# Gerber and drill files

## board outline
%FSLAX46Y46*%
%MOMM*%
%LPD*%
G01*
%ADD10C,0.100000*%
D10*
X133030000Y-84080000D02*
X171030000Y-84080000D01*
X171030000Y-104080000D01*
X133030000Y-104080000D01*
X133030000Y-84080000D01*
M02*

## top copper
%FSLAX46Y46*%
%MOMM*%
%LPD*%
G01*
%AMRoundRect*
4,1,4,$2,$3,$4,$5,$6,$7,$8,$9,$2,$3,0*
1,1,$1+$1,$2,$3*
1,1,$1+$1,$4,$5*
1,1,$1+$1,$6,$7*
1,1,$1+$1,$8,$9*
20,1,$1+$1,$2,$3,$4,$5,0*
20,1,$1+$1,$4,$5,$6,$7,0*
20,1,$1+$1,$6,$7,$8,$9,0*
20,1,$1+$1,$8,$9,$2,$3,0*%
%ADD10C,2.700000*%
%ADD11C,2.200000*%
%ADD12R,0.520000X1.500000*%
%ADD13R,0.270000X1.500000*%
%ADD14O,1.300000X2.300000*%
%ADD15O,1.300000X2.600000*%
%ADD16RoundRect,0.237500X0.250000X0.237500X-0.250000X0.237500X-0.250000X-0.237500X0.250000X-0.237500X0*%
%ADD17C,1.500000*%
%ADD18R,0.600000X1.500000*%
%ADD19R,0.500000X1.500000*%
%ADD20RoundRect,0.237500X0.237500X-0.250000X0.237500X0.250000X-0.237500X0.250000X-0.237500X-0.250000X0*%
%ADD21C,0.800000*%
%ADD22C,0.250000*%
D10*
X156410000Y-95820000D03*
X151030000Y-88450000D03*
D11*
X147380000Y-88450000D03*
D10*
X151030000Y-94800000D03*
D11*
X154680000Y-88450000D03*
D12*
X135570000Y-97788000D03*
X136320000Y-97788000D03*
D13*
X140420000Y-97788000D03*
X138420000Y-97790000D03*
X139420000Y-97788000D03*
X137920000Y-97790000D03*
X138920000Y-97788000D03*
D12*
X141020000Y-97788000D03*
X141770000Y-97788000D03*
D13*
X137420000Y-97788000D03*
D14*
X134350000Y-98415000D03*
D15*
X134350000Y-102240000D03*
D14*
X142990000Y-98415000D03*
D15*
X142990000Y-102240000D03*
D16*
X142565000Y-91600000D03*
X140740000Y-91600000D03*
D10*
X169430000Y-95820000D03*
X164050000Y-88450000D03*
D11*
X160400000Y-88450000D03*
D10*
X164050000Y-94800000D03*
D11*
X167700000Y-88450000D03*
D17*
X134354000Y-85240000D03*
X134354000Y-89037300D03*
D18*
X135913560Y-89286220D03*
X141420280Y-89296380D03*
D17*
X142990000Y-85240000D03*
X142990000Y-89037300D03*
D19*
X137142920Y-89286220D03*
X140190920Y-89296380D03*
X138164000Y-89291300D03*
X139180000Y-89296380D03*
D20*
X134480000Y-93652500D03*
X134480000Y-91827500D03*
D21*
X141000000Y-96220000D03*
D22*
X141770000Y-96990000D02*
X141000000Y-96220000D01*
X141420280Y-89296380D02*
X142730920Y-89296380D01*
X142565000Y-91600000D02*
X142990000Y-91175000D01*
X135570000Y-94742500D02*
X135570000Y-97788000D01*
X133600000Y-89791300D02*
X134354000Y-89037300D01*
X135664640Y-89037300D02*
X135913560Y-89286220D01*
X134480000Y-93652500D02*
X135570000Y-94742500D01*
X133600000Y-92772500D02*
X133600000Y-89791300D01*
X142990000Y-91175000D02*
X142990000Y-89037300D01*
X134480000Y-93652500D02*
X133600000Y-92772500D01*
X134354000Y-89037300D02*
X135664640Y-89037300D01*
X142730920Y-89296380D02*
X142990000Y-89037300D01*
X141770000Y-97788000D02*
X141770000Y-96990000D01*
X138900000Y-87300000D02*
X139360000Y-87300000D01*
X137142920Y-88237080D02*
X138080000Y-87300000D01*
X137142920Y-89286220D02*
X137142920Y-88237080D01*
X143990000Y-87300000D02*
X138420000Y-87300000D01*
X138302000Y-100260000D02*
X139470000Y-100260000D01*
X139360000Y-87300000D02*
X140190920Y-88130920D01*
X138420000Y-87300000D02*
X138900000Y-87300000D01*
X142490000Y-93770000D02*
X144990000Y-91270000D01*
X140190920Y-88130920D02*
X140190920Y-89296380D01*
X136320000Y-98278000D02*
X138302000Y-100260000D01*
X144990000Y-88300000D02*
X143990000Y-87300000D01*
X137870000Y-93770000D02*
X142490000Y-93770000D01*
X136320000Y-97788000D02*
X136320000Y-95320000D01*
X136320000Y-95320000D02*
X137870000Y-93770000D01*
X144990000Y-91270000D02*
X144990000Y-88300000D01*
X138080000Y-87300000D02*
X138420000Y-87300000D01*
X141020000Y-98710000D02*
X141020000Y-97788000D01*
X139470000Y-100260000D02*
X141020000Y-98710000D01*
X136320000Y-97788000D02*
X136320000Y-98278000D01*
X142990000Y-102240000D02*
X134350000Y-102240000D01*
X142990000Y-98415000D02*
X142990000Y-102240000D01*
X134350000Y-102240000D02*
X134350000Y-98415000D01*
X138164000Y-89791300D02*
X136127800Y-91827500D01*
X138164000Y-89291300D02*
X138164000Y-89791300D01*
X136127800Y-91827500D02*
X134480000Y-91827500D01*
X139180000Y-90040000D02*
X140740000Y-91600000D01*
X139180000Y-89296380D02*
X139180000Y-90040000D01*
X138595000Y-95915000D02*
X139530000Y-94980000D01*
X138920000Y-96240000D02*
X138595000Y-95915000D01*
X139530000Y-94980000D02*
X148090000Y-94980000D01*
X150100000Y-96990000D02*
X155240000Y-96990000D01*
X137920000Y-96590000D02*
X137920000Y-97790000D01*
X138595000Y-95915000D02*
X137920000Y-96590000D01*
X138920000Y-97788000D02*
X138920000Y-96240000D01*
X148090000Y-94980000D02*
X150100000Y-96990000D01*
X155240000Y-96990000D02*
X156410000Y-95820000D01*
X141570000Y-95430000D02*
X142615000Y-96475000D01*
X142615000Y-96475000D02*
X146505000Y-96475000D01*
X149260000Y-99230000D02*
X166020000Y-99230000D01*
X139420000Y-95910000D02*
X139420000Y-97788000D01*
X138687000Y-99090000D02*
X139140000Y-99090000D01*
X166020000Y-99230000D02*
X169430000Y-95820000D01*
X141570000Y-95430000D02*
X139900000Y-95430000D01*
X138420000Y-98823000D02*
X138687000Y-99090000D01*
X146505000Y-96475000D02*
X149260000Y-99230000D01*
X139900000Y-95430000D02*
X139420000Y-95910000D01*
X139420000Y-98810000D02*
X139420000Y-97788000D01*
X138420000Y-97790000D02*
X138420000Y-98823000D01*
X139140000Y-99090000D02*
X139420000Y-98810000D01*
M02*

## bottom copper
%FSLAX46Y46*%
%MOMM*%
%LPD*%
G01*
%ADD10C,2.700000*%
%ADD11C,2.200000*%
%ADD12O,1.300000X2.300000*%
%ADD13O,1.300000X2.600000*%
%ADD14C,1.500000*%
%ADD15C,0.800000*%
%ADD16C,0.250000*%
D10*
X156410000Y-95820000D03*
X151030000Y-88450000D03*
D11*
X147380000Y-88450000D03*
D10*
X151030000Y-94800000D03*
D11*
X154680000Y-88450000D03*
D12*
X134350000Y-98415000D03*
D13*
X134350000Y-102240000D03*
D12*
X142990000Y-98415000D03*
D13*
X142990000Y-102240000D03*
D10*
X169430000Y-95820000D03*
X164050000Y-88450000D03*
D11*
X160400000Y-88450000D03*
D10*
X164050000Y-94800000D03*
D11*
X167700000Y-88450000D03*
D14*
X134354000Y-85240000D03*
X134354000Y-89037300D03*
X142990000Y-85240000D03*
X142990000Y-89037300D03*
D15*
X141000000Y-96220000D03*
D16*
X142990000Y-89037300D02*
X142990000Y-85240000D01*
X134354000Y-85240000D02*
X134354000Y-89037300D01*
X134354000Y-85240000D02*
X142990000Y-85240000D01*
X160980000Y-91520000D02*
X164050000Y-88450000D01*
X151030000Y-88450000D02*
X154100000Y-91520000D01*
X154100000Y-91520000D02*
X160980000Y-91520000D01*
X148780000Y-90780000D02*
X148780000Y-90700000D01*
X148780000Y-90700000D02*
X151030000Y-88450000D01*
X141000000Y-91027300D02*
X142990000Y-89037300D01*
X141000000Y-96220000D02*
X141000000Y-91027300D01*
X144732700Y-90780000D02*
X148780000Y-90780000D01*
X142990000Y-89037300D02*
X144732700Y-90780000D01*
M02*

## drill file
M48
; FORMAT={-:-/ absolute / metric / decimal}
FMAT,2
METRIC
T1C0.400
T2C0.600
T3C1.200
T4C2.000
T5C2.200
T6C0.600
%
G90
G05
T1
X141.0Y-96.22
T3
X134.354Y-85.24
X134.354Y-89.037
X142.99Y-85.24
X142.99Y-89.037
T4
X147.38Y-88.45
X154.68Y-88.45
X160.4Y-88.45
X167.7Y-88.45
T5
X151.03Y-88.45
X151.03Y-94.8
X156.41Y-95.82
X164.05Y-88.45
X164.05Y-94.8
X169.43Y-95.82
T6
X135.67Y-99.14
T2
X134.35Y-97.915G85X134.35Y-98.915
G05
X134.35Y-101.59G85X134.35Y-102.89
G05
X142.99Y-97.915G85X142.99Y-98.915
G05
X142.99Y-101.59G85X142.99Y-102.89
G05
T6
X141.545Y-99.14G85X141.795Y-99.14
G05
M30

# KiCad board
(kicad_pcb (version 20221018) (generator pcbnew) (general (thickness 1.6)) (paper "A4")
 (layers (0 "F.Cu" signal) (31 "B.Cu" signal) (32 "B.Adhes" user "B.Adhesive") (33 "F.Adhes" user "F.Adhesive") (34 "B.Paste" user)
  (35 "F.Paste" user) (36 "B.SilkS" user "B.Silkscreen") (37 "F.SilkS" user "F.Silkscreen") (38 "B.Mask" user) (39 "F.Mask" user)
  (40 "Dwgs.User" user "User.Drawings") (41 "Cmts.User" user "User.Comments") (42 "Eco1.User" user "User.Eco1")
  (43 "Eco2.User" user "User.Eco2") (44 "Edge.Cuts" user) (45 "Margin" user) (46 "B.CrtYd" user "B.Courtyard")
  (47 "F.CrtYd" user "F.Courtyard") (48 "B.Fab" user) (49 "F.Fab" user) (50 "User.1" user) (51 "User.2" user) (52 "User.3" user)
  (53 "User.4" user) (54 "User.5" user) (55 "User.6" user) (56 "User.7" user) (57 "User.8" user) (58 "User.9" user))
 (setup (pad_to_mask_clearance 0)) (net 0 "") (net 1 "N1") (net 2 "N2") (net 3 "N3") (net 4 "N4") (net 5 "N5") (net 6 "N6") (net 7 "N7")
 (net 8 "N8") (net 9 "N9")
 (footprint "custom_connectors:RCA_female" (layer "F.Cu") (at 151.03 88.45)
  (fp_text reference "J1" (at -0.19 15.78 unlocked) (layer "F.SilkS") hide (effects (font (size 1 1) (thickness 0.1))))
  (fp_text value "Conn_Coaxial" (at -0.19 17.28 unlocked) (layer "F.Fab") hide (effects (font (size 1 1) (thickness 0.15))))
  (pad "1" thru_hole circle (at 5.38 7.37) (size 2.7 2.7) (drill 2.2) (layers "*.Cu" "*.Mask") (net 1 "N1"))
  (pad "2" thru_hole circle (at 0 0) (size 2.7 2.7) (drill 2.2) (layers "*.Cu" "*.Mask") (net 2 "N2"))
  (pad "3" thru_hole circle (at -3.65 0) (size 2.2 2.2) (drill 2) (layers "*.Cu" "*.Mask"))
  (pad "3" thru_hole circle (at 0 6.35) (size 2.7 2.7) (drill 2.2) (layers "*.Cu" "*.Mask"))
  (pad "3" thru_hole circle (at 3.65 0) (size 2.2 2.2) (drill 2) (layers "*.Cu" "*.Mask")))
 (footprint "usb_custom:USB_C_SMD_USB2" (layer "F.Cu") (at 138.67 101.09)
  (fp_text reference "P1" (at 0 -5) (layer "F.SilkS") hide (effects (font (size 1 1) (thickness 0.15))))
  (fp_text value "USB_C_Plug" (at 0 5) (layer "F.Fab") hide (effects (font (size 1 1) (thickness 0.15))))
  (pad "" np_thru_hole circle (at -3 -1.95) (size 0.6 0.6) (drill 0.6) (layers "F&B.Cu" "*.Mask"))
  (pad "" np_thru_hole oval (at 3 -1.95) (size 0.85 0.6) (drill oval 0.85 0.6) (layers "F&B.Cu" "*.Mask"))
  (pad "A1" smd rect (at -3.1 -3.302) (size 0.52 1.5) (layers "F.Cu" "F.Paste" "F.Mask") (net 2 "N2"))
  (pad "A4" smd rect (at -2.35 -3.302) (size 0.52 1.5) (layers "F.Cu" "F.Paste" "F.Mask") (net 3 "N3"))
  (pad "A5" smd rect (at 1.75 -3.302) (size 0.27 1.5) (layers "F.Cu" "F.Paste" "F.Mask") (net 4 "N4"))
  (pad "A6" smd rect (at -0.25 -3.3) (size 0.27 1.5) (layers "F.Cu" "F.Paste" "F.Mask") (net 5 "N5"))
  (pad "A6" smd rect (at 0.75 -3.302) (size 0.27 1.5) (layers "F.Cu" "F.Paste" "F.Mask") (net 5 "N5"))
  (pad "A7" smd rect (at -0.75 -3.3) (size 0.27 1.5) (layers "F.Cu" "F.Paste" "F.Mask") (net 1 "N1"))
  (pad "A7" smd rect (at 0.25 -3.302) (size 0.27 1.5) (layers "F.Cu" "F.Paste" "F.Mask") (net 1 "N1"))
  (pad "A9" smd rect (at 2.35 -3.302) (size 0.52 1.5) (layers "F.Cu" "F.Paste" "F.Mask") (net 3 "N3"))
  (pad "A12" smd rect (at 3.1 -3.302) (size 0.52 1.5) (layers "F.Cu" "F.Paste" "F.Mask") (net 2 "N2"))
  (pad "B5" smd rect (at -1.25 -3.302) (size 0.27 1.5) (layers "F.Cu" "F.Paste" "F.Mask") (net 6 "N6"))
  (pad "S1" thru_hole oval (at -4.32 -2.675) (size 1.3 2.3) (drill oval 0.6 1.6) (layers "*.Cu" "*.Mask") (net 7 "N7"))
  (pad "S1" thru_hole oval (at -4.32 1.15) (size 1.3 2.6) (drill oval 0.6 1.9) (layers "*.Cu" "*.Mask") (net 7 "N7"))
  (pad "S1" thru_hole oval (at 4.32 -2.675) (size 1.3 2.3) (drill oval 0.6 1.6) (layers "*.Cu" "*.Mask") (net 7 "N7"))
  (pad "S1" thru_hole oval (at 4.32 1.15) (size 1.3 2.6) (drill oval 0.6 1.9) (layers "*.Cu" "*.Mask") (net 7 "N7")))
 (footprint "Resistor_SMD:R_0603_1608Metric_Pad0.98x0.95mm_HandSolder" (layer "F.Cu") (at 141.6525 91.6 180)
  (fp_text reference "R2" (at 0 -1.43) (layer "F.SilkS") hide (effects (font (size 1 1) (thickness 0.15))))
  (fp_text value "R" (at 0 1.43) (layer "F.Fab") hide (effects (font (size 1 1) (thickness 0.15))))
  (pad "1" smd roundrect (at -0.9125 0 180) (size 0.975 0.95) (layers "F.Cu" "F.Paste" "F.Mask") (roundrect_rratio 0.25) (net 2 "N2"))
  (pad "2" smd roundrect (at 0.9125 0 180) (size 0.975 0.95) (layers "F.Cu" "F.Paste" "F.Mask") (roundrect_rratio 0.25) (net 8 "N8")))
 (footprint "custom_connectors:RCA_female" (layer "F.Cu") (at 164.05 88.45)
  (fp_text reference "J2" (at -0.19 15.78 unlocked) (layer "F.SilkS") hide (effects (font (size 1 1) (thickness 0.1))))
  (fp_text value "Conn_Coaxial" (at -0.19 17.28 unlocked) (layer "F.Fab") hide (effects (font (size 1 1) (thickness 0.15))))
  (pad "1" thru_hole circle (at 5.38 7.37) (size 2.7 2.7) (drill 2.2) (layers "*.Cu" "*.Mask") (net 5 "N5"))
  (pad "2" thru_hole circle (at 0 0) (size 2.7 2.7) (drill 2.2) (layers "*.Cu" "*.Mask") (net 2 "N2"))
  (pad "3" thru_hole circle (at -3.65 0) (size 2.2 2.2) (drill 2) (layers "*.Cu" "*.Mask"))
  (pad "3" thru_hole circle (at 0 6.35) (size 2.7 2.7) (drill 2.2) (layers "*.Cu" "*.Mask"))
  (pad "3" thru_hole circle (at 3.65 0) (size 2.2 2.2) (drill 2) (layers "*.Cu" "*.Mask")))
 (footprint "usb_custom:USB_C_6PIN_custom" (layer "F.Cu") (at 138.672 89.0373)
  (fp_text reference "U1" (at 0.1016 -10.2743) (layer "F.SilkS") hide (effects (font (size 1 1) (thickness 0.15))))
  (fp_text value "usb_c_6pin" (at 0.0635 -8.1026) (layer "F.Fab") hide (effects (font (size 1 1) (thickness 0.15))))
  (pad "1" thru_hole circle (at -4.318 -3.7973) (size 1.5 1.5) (drill 1.2) (layers "*.Cu" "*.Mask") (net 2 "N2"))
  (pad "1" thru_hole circle (at -4.318 0) (size 1.5 1.5) (drill 1.2) (layers "*.Cu" "*.Mask") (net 2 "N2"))
  (pad "1" smd rect (at -2.75844 0.24892) (size 0.6 1.5) (layers "F.Cu" "F.Paste" "F.Mask") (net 2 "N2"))
  (pad "1" smd rect (at 2.74828 0.25908) (size 0.6 1.5) (layers "F.Cu" "F.Paste" "F.Mask") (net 2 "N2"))
  (pad "1" thru_hole circle (at 4.318 -3.7973) (size 1.5 1.5) (drill 1.2) (layers "*.Cu" "*.Mask") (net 2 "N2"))
  (pad "1" thru_hole circle (at 4.318 0) (size 1.5 1.5) (drill 1.2) (layers "*.Cu" "*.Mask") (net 2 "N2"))
  (pad "2" smd rect (at -1.52908 0.24892) (size 0.5 1.5) (layers "F.Cu" "F.Paste" "F.Mask") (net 3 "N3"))
  (pad "2" smd rect (at 1.51892 0.25908) (size 0.5 1.5) (layers "F.Cu" "F.Paste" "F.Mask") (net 3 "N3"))
  (pad "3" smd rect (at -0.508 0.254) (size 0.5 1.5) (layers "F.Cu" "F.Paste" "F.Mask") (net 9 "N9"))
  (pad "4" smd rect (at 0.508 0.25908) (size 0.5 1.5) (layers "F.Cu" "F.Paste" "F.Mask") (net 8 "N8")))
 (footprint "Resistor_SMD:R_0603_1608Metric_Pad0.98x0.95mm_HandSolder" (layer "F.Cu") (at 134.48 92.74 90)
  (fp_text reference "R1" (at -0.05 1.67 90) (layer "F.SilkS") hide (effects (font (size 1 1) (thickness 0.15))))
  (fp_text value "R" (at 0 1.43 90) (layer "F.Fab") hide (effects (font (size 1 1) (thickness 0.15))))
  (pad "1" smd roundrect (at -0.9125 0 90) (size 0.975 0.95) (layers "F.Cu" "F.Paste" "F.Mask") (roundrect_rratio 0.25) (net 2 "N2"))
  (pad "2" smd roundrect (at 0.9125 0 90) (size 0.975 0.95) (layers "F.Cu" "F.Paste" "F.Mask") (roundrect_rratio 0.25) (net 9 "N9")))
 (gr_rect (start 133.03 84.08) (end 171.03 104.08) (stroke (width 0.1) (type default)) (fill none) (layer "Edge.Cuts"))
 (segment (start 141.77 96.99) (end 141 96.22) (width 0.25) (layer "F.Cu") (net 2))
 (segment (start 141.42028 89.29638) (end 142.73092 89.29638) (width 0.25) (layer "F.Cu") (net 2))
 (segment (start 142.565 91.6) (end 142.99 91.175) (width 0.25) (layer "F.Cu") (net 2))
 (segment (start 135.57 94.7425) (end 135.57 97.788) (width 0.25) (layer "F.Cu") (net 2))
 (segment (start 133.6 89.7913) (end 134.354 89.0373) (width 0.25) (layer "F.Cu") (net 2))
 (segment (start 135.66464 89.0373) (end 135.91356 89.28622) (width 0.25) (layer "F.Cu") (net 2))
 (segment (start 134.48 93.6525) (end 135.57 94.7425) (width 0.25) (layer "F.Cu") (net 2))
 (segment (start 133.6 92.7725) (end 133.6 89.7913) (width 0.25) (layer "F.Cu") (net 2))
 (segment (start 142.99 91.175) (end 142.99 89.0373) (width 0.25) (layer "F.Cu") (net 2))
 (segment (start 134.48 93.6525) (end 133.6 92.7725) (width 0.25) (layer "F.Cu") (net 2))
 (segment (start 134.354 89.0373) (end 135.66464 89.0373) (width 0.25) (layer "F.Cu") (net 2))
 (segment (start 142.73092 89.29638) (end 142.99 89.0373) (width 0.25) (layer "F.Cu") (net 2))
 (segment (start 141.77 97.788) (end 141.77 96.99) (width 0.25) (layer "F.Cu") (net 2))
 (via (at 141 96.22) (size 0.8) (drill 0.4) (layers "F.Cu" "B.Cu") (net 2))
 (segment (start 142.99 89.0373) (end 142.99 85.24) (width 0.25) (layer "B.Cu") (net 2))
 (segment (start 134.354 85.24) (end 134.354 89.0373) (width 0.25) (layer "B.Cu") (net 2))
 (segment (start 134.354 85.24) (end 142.99 85.24) (width 0.25) (layer "B.Cu") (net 2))
 (segment (start 160.98 91.52) (end 164.05 88.45) (width 0.25) (layer "B.Cu") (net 2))
 (segment (start 151.03 88.45) (end 154.1 91.52) (width 0.25) (layer "B.Cu") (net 2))
 (segment (start 154.1 91.52) (end 160.98 91.52) (width 0.25) (layer "B.Cu") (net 2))
 (segment (start 148.78 90.78) (end 148.78 90.7) (width 0.25) (layer "B.Cu") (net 2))
 (segment (start 148.78 90.7) (end 151.03 88.45) (width 0.25) (layer "B.Cu") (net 2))
 (segment (start 141 91.0273) (end 142.99 89.0373) (width 0.25) (layer "B.Cu") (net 2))
 (segment (start 141 96.22) (end 141 91.0273) (width 0.25) (layer "B.Cu") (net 2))
 (segment (start 144.7327 90.78) (end 148.78 90.78) (width 0.25) (layer "B.Cu") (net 2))
 (segment (start 142.99 89.0373) (end 144.7327 90.78) (width 0.25) (layer "B.Cu") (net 2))
 (segment (start 138.9 87.3) (end 139.36 87.3) (width 0.25) (layer "F.Cu") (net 3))
 (segment (start 137.14292 88.23708) (end 138.08 87.3) (width 0.25) (layer "F.Cu") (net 3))
 (segment (start 137.14292 89.28622) (end 137.14292 88.23708) (width 0.25) (layer "F.Cu") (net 3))
 (segment (start 143.99 87.3) (end 138.42 87.3) (width 0.25) (layer "F.Cu") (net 3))
 (segment (start 138.302 100.26) (end 139.47 100.26) (width 0.25) (layer "F.Cu") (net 3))
 (segment (start 139.36 87.3) (end 140.19092 88.13092) (width 0.25) (layer "F.Cu") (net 3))
 (segment (start 138.42 87.3) (end 138.9 87.3) (width 0.25) (layer "F.Cu") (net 3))
 (segment (start 142.49 93.77) (end 144.99 91.27) (width 0.25) (layer "F.Cu") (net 3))
 (segment (start 140.19092 88.13092) (end 140.19092 89.29638) (width 0.25) (layer "F.Cu") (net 3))
 (segment (start 136.32 98.278) (end 138.302 100.26) (width 0.25) (layer "F.Cu") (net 3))
 (segment (start 144.99 88.3) (end 143.99 87.3) (width 0.25) (layer "F.Cu") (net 3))
 (segment (start 137.87 93.77) (end 142.49 93.77) (width 0.25) (layer "F.Cu") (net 3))
 (segment (start 136.32 97.788) (end 136.32 95.32) (width 0.25) (layer "F.Cu") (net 3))
 (segment (start 136.32 95.32) (end 137.87 93.77) (width 0.25) (layer "F.Cu") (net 3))
 (segment (start 144.99 91.27) (end 144.99 88.3) (width 0.25) (layer "F.Cu") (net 3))
 (segment (start 138.08 87.3) (end 138.42 87.3) (width 0.25) (layer "F.Cu") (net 3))
 (segment (start 141.02 98.71) (end 141.02 97.788) (width 0.25) (layer "F.Cu") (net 3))
 (segment (start 139.47 100.26) (end 141.02 98.71) (width 0.25) (layer "F.Cu") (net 3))
 (segment (start 136.32 97.788) (end 136.32 98.278) (width 0.25) (layer "F.Cu") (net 3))
 (segment (start 142.99 102.24) (end 134.35 102.24) (width 0.25) (layer "F.Cu") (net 7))
 (segment (start 142.99 98.415) (end 142.99 102.24) (width 0.25) (layer "F.Cu") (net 7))
 (segment (start 134.35 102.24) (end 134.35 98.415) (width 0.25) (layer "F.Cu") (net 7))
 (segment (start 138.164 89.7913) (end 136.1278 91.8275) (width 0.25) (layer "F.Cu") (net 9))
 (segment (start 138.164 89.2913) (end 138.164 89.7913) (width 0.25) (layer "F.Cu") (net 9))
 (segment (start 136.1278 91.8275) (end 134.48 91.8275) (width 0.25) (layer "F.Cu") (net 9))
 (segment (start 139.18 90.04) (end 140.74 91.6) (width 0.25) (layer "F.Cu") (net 8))
 (segment (start 139.18 89.29638) (end 139.18 90.04) (width 0.25) (layer "F.Cu") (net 8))
 (segment (start 138.595 95.915) (end 139.53 94.98) (width 0.25) (layer "F.Cu") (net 1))
 (segment (start 138.92 96.24) (end 138.595 95.915) (width 0.25) (layer "F.Cu") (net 1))
 (segment (start 139.53 94.98) (end 148.09 94.98) (width 0.25) (layer "F.Cu") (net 1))
 (segment (start 150.1 96.99) (end 155.24 96.99) (width 0.25) (layer "F.Cu") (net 1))
 (segment (start 137.92 96.59) (end 137.92 97.79) (width 0.25) (layer "F.Cu") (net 1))
 (segment (start 138.595 95.915) (end 137.92 96.59) (width 0.25) (layer "F.Cu") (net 1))
 (segment (start 138.92 97.788) (end 138.92 96.24) (width 0.25) (layer "F.Cu") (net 1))
 (segment (start 148.09 94.98) (end 150.1 96.99) (width 0.25) (layer "F.Cu") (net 1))
 (segment (start 155.24 96.99) (end 156.41 95.82) (width 0.25) (layer "F.Cu") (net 1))
 (segment (start 141.57 95.43) (end 142.615 96.475) (width 0.25) (layer "F.Cu") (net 5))
 (segment (start 142.615 96.475) (end 146.505 96.475) (width 0.25) (layer "F.Cu") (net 5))
 (segment (start 149.26 99.23) (end 166.02 99.23) (width 0.25) (layer "F.Cu") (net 5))
 (segment (start 139.42 95.91) (end 139.42 97.788) (width 0.25) (layer "F.Cu") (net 5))
 (segment (start 138.687 99.09) (end 139.14 99.09) (width 0.25) (layer "F.Cu") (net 5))
 (segment (start 166.02 99.23) (end 169.43 95.82) (width 0.25) (layer "F.Cu") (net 5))
 (segment (start 141.57 95.43) (end 139.9 95.43) (width 0.25) (layer "F.Cu") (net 5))
 (segment (start 138.42 98.823) (end 138.687 99.09) (width 0.25) (layer "F.Cu") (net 5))
 (segment (start 146.505 96.475) (end 149.26 99.23) (width 0.25) (layer "F.Cu") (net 5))
 (segment (start 139.9 95.43) (end 139.42 95.91) (width 0.25) (layer "F.Cu") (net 5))
 (segment (start 139.42 98.81) (end 139.42 97.788) (width 0.25) (layer "F.Cu") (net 5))
 (segment (start 138.42 97.79) (end 138.42 98.823) (width 0.25) (layer "F.Cu") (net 5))
 (segment (start 139.14 99.09) (end 139.42 98.81) (width 0.25) (layer "F.Cu") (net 5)))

